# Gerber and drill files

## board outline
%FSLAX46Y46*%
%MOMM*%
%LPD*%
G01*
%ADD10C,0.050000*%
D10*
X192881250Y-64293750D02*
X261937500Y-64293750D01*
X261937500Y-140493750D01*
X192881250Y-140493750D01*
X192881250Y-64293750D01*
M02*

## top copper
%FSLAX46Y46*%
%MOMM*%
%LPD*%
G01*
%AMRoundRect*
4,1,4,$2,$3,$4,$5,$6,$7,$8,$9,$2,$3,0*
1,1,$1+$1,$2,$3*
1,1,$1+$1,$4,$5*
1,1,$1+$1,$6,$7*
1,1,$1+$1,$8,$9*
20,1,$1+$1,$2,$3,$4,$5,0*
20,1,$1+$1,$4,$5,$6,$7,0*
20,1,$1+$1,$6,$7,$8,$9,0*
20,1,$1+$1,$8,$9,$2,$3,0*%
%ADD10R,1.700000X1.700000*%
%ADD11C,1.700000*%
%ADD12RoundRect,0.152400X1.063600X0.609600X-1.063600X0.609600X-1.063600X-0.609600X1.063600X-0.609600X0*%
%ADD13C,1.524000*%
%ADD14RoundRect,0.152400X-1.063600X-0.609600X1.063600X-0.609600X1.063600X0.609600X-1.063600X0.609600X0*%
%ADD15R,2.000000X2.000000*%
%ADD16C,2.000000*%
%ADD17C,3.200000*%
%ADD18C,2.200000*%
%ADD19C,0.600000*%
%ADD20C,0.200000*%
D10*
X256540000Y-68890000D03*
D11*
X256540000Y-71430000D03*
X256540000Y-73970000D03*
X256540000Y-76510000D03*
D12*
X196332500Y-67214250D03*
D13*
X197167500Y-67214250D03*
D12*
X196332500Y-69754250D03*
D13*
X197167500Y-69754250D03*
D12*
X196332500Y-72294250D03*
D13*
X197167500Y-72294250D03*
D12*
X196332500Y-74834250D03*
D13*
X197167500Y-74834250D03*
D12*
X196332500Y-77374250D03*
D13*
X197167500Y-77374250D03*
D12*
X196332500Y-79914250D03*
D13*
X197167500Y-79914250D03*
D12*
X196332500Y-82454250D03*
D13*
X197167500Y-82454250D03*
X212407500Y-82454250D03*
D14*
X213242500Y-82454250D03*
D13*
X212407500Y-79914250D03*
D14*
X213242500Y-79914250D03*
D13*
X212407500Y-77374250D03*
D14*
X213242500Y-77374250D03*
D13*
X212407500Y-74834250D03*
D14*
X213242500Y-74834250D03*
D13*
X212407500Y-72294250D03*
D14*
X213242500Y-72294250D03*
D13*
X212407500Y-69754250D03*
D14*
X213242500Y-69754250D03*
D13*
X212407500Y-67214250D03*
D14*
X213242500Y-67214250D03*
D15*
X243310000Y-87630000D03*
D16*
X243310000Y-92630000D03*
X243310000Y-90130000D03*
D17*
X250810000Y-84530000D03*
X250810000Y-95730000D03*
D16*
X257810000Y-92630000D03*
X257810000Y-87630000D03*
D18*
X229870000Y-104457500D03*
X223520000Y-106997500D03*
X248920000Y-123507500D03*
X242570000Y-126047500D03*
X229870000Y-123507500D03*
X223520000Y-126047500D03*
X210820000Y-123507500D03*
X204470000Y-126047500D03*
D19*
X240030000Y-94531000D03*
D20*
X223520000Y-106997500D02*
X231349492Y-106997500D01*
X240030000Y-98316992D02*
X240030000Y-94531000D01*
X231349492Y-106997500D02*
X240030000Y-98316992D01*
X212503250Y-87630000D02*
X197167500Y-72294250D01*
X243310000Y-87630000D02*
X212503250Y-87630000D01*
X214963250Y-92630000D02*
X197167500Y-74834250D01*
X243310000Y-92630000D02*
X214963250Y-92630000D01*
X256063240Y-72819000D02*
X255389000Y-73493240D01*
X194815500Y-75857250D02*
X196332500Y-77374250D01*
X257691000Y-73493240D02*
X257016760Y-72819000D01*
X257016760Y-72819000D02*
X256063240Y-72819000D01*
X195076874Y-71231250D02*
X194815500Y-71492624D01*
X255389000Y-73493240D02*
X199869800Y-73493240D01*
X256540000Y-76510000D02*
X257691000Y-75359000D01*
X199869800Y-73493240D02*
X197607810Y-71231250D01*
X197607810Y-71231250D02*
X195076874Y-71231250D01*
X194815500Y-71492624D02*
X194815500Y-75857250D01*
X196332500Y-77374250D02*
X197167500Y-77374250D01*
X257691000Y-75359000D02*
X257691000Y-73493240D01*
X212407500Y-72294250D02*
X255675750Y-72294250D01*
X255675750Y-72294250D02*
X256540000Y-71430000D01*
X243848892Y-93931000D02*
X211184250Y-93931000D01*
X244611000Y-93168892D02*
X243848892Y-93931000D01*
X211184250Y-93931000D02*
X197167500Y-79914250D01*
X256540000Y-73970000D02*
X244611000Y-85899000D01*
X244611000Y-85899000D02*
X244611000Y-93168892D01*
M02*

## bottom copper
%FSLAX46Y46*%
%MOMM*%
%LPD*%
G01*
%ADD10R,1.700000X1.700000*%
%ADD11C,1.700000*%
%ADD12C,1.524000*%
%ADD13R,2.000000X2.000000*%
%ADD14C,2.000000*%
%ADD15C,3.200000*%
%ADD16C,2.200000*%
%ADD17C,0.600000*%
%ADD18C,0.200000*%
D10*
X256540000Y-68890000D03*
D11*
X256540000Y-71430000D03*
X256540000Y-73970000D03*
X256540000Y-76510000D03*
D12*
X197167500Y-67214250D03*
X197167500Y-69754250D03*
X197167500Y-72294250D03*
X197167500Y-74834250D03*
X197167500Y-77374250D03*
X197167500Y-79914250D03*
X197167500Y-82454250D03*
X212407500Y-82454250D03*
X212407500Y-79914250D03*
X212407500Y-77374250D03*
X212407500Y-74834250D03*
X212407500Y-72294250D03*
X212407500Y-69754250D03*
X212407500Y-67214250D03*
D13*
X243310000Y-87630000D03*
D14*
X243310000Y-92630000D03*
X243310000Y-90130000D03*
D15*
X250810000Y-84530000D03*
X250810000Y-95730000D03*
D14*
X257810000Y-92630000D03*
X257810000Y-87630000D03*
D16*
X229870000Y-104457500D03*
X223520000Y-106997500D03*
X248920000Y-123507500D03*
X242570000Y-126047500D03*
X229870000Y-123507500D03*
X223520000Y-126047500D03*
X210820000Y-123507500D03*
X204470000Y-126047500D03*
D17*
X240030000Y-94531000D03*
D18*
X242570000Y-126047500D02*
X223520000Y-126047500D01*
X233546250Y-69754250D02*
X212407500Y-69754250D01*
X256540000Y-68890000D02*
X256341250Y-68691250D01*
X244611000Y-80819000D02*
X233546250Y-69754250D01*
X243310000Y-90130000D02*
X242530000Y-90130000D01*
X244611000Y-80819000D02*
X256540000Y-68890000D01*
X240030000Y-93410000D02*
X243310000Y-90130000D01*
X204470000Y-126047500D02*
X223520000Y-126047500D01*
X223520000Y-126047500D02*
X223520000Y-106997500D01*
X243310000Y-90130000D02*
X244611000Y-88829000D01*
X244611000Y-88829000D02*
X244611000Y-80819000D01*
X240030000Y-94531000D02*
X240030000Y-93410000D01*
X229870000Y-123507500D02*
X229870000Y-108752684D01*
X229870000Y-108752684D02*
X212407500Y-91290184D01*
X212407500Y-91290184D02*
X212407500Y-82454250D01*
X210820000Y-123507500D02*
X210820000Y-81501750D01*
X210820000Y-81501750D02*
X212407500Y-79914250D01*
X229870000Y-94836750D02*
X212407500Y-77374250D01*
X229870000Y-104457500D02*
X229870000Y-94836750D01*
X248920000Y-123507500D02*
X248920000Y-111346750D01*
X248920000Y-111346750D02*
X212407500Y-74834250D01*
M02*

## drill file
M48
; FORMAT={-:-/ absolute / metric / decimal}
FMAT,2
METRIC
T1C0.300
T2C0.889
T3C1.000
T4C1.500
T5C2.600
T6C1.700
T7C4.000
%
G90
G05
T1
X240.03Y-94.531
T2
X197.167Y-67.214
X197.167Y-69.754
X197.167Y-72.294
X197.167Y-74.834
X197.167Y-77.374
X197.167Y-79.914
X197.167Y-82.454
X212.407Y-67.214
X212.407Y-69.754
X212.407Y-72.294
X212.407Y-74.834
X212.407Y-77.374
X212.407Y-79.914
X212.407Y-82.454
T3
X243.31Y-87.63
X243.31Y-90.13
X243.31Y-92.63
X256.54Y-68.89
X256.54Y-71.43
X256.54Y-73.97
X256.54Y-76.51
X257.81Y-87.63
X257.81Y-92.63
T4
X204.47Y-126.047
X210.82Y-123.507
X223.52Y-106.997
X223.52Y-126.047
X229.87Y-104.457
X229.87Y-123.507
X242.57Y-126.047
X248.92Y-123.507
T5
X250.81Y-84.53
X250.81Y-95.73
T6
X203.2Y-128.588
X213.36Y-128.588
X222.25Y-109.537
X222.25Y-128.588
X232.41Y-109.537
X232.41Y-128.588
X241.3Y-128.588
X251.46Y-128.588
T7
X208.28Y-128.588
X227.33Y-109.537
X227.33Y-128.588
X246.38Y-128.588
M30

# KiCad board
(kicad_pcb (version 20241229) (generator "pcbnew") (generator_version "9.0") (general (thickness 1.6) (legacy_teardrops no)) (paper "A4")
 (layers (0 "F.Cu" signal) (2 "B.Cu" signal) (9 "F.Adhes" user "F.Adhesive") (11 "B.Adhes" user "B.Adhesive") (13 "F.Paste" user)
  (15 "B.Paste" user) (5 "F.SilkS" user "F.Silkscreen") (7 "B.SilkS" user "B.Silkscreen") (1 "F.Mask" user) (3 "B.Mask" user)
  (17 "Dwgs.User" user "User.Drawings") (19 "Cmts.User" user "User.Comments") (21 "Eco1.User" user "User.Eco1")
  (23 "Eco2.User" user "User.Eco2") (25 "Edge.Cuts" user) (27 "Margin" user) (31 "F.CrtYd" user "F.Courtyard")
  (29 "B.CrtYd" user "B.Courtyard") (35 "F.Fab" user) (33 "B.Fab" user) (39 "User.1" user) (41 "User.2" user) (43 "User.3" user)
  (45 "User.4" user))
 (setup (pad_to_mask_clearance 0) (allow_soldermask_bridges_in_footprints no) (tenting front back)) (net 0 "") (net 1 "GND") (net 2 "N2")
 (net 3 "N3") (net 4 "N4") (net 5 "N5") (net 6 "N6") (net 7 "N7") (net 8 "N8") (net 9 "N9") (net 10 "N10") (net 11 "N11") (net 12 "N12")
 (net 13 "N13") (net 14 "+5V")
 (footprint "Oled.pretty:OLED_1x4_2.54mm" (layer "F.Cu") (at 256.54 68.89 -90)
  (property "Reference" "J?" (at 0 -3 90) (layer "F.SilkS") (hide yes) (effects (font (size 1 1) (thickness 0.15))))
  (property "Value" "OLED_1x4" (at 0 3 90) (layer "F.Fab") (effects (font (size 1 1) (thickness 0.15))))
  (pad "1" thru_hole rect (at 0 0 270) (size 1.7 1.7) (drill 1) (layers "*.Cu" "*.Mask") (remove_unused_layers no) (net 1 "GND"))
  (pad "2" thru_hole circle (at 2.54 0 270) (size 1.7 1.7) (drill 1) (layers "*.Cu" "*.Mask") (remove_unused_layers no) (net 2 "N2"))
  (pad "3" thru_hole circle (at 5.08 0 270) (size 1.7 1.7) (drill 1) (layers "*.Cu" "*.Mask") (remove_unused_layers no) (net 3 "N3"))
  (pad "4" thru_hole circle (at 7.62 0 270) (size 1.7 1.7) (drill 1) (layers "*.Cu" "*.Mask") (remove_unused_layers no) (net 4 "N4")))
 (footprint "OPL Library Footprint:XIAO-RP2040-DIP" (layer "F.Cu") (at 204.7875 74.83425)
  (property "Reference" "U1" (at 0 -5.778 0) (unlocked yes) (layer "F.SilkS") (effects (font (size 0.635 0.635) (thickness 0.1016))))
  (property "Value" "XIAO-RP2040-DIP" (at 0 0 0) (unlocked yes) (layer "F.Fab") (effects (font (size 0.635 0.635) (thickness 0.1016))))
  (pad "1" smd roundrect (at -8.455 -7.62 180) (size 2.432 1.524) (layers "F.Cu" "F.Mask") (roundrect_rratio 0.1) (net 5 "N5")
   (thermal_bridge_angle 45))
  (pad "1" thru_hole circle (at -7.62 -7.62 180) (size 1.524 1.524) (drill 0.889) (layers "*.Cu" "*.Mask") (remove_unused_layers no)
   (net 5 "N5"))
  (pad "2" smd roundrect (at -8.455 -5.08 180) (size 2.432 1.524) (layers "F.Cu" "F.Mask") (roundrect_rratio 0.1) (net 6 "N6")
   (thermal_bridge_angle 45))
  (pad "2" thru_hole circle (at -7.62 -5.08 180) (size 1.524 1.524) (drill 0.889) (layers "*.Cu" "*.Mask") (remove_unused_layers no)
   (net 6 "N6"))
  (pad "3" smd roundrect (at -8.455 -2.54 180) (size 2.432 1.524) (layers "F.Cu" "F.Mask") (roundrect_rratio 0.1) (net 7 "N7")
   (thermal_bridge_angle 45))
  (pad "3" thru_hole circle (at -7.62 -2.54 180) (size 1.524 1.524) (drill 0.889) (layers "*.Cu" "*.Mask") (remove_unused_layers no)
   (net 7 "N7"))
  (pad "4" smd roundrect (at -8.455 0 180) (size 2.432 1.524) (layers "F.Cu" "F.Mask") (roundrect_rratio 0.1) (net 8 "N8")
   (thermal_bridge_angle 45))
  (pad "4" thru_hole circle (at -7.62 0 180) (size 1.524 1.524) (drill 0.889) (layers "*.Cu" "*.Mask") (remove_unused_layers no)
   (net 8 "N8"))
  (pad "5" smd roundrect (at -8.455 2.54 180) (size 2.432 1.524) (layers "F.Cu" "F.Mask") (roundrect_rratio 0.1) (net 4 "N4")
   (thermal_bridge_angle 45))
  (pad "5" thru_hole circle (at -7.62 2.54 180) (size 1.524 1.524) (drill 0.889) (layers "*.Cu" "*.Mask") (remove_unused_layers no)
   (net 4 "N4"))
  (pad "6" smd roundrect (at -8.455 5.08 180) (size 2.432 1.524) (layers "F.Cu" "F.Mask") (roundrect_rratio 0.1) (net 3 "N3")
   (thermal_bridge_angle 45))
  (pad "6" thru_hole circle (at -7.62 5.08 180) (size 1.524 1.524) (drill 0.889) (layers "*.Cu" "*.Mask") (remove_unused_layers no)
   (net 3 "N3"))
  (pad "7" smd roundrect (at -8.455 7.62 180) (size 2.432 1.524) (layers "F.Cu" "F.Mask") (roundrect_rratio 0.1) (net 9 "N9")
   (thermal_bridge_angle 45))
  (pad "7" thru_hole circle (at -7.62 7.62 180) (size 1.524 1.524) (drill 0.889) (layers "*.Cu" "*.Mask") (remove_unused_layers no)
   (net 9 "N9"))
  (pad "8" thru_hole circle (at 7.62 7.62) (size 1.524 1.524) (drill 0.889) (layers "*.Cu" "*.Mask") (remove_unused_layers no)
   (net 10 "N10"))
  (pad "8" smd roundrect (at 8.455 7.62) (size 2.432 1.524) (layers "F.Cu" "F.Mask") (roundrect_rratio 0.1) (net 10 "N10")
   (thermal_bridge_angle 45))
  (pad "9" thru_hole circle (at 7.62 5.08) (size 1.524 1.524) (drill 0.889) (layers "*.Cu" "*.Mask") (remove_unused_layers no)
   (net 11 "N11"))
  (pad "9" smd roundrect (at 8.455 5.08) (size 2.432 1.524) (layers "F.Cu" "F.Mask") (roundrect_rratio 0.1) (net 11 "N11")
   (thermal_bridge_angle 45))
  (pad "10" thru_hole circle (at 7.62 2.54) (size 1.524 1.524) (drill 0.889) (layers "*.Cu" "*.Mask") (remove_unused_layers no)
   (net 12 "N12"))
  (pad "10" smd roundrect (at 8.455 2.54) (size 2.432 1.524) (layers "F.Cu" "F.Mask") (roundrect_rratio 0.1) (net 12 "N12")
   (thermal_bridge_angle 45))
  (pad "11" thru_hole circle (at 7.62 0) (size 1.524 1.524) (drill 0.889) (layers "*.Cu" "*.Mask") (remove_unused_layers no) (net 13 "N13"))
  (pad "11" smd roundrect (at 8.455 0) (size 2.432 1.524) (layers "F.Cu" "F.Mask") (roundrect_rratio 0.1) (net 13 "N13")
   (thermal_bridge_angle 45))
  (pad "12" thru_hole circle (at 7.62 -2.54) (size 1.524 1.524) (drill 0.889) (layers "*.Cu" "*.Mask") (remove_unused_layers no)
   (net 2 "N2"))
  (pad "12" smd roundrect (at 8.455 -2.54) (size 2.432 1.524) (layers "F.Cu" "F.Mask") (roundrect_rratio 0.1) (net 2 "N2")
   (thermal_bridge_angle 45))
  (pad "13" thru_hole circle (at 7.62 -5.08) (size 1.524 1.524) (drill 0.889) (layers "*.Cu" "*.Mask") (remove_unused_layers no)
   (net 1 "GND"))
  (pad "13" smd roundrect (at 8.455 -5.08) (size 2.432 1.524) (layers "F.Cu" "F.Mask") (roundrect_rratio 0.1) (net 1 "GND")
   (thermal_bridge_angle 45))
  (pad "14" thru_hole circle (at 7.62 -7.62) (size 1.524 1.524) (drill 0.889) (layers "*.Cu" "*.Mask") (remove_unused_layers no)
   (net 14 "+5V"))
  (pad "14" smd roundrect (at 8.455 -7.62) (size 2.432 1.524) (layers "F.Cu" "F.Mask") (roundrect_rratio 0.1) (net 14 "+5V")
   (thermal_bridge_angle 45)))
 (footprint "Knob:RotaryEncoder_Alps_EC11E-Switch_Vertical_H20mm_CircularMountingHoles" (layer "F.Cu") (at 243.31 87.63)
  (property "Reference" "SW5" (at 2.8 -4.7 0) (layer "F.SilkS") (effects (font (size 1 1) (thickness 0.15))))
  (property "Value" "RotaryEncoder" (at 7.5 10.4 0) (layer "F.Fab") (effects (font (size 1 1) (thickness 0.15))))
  (pad "A" thru_hole rect (at 0 0) (size 2 2) (drill 1) (layers "*.Cu" "*.Mask") (remove_unused_layers no) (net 7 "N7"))
  (pad "B" thru_hole circle (at 0 5) (size 2 2) (drill 1) (layers "*.Cu" "*.Mask") (remove_unused_layers no) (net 8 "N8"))
  (pad "C" thru_hole circle (at 0 2.5) (size 2 2) (drill 1) (layers "*.Cu" "*.Mask") (remove_unused_layers no) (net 1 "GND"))
  (pad "MP" thru_hole circle (at 7.5 -3.1) (size 3.2 3.2) (drill 2.6) (layers "*.Cu" "*.Mask") (remove_unused_layers no))
  (pad "MP" thru_hole circle (at 7.5 8.1) (size 3.2 3.2) (drill 2.6) (layers "*.Cu" "*.Mask") (remove_unused_layers no))
  (pad "S1" thru_hole circle (at 14.5 5) (size 2 2) (drill 1) (layers "*.Cu" "*.Mask") (remove_unused_layers no))
  (pad "S2" thru_hole circle (at 14.5 0) (size 2 2) (drill 1) (layers "*.Cu" "*.Mask") (remove_unused_layers no)))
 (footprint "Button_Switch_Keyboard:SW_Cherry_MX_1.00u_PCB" (layer "F.Cu") (at 229.87 104.4575)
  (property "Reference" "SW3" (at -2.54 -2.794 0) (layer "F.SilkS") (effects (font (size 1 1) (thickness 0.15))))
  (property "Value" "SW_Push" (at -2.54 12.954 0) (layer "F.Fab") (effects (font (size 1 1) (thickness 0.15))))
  (pad "" np_thru_hole circle (at -7.62 5.08) (size 1.7 1.7) (drill 1.7) (layers "*.Cu" "*.Mask"))
  (pad "" np_thru_hole circle (at -2.54 5.08) (size 4 4) (drill 4) (layers "*.Cu" "*.Mask"))
  (pad "" np_thru_hole circle (at 2.54 5.08) (size 1.7 1.7) (drill 1.7) (layers "*.Cu" "*.Mask"))
  (pad "1" thru_hole circle (at 0 0) (size 2.2 2.2) (drill 1.5) (layers "*.Cu" "*.Mask") (remove_unused_layers no) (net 12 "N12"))
  (pad "2" thru_hole circle (at -6.35 2.54) (size 2.2 2.2) (drill 1.5) (layers "*.Cu" "*.Mask") (remove_unused_layers no) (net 1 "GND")))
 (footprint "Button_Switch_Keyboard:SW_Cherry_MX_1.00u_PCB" (layer "F.Cu") (at 248.92 123.5075)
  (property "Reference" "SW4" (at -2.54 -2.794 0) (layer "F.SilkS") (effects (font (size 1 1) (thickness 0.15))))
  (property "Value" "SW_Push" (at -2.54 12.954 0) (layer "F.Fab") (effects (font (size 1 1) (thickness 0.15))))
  (pad "" np_thru_hole circle (at -7.62 5.08) (size 1.7 1.7) (drill 1.7) (layers "*.Cu" "*.Mask"))
  (pad "" np_thru_hole circle (at -2.54 5.08) (size 4 4) (drill 4) (layers "*.Cu" "*.Mask"))
  (pad "" np_thru_hole circle (at 2.54 5.08) (size 1.7 1.7) (drill 1.7) (layers "*.Cu" "*.Mask"))
  (pad "1" thru_hole circle (at 0 0) (size 2.2 2.2) (drill 1.5) (layers "*.Cu" "*.Mask") (remove_unused_layers no) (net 13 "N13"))
  (pad "2" thru_hole circle (at -6.35 2.54) (size 2.2 2.2) (drill 1.5) (layers "*.Cu" "*.Mask") (remove_unused_layers no) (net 1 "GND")))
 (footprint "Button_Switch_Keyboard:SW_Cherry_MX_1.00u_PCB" (layer "F.Cu") (at 229.87 123.5075)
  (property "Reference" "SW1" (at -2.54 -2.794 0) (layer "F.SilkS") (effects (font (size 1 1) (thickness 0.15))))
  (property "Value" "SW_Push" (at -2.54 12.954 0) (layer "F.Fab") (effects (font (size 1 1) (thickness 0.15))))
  (pad "" np_thru_hole circle (at -7.62 5.08) (size 1.7 1.7) (drill 1.7) (layers "*.Cu" "*.Mask"))
  (pad "" np_thru_hole circle (at -2.54 5.08) (size 4 4) (drill 4) (layers "*.Cu" "*.Mask"))
  (pad "" np_thru_hole circle (at 2.54 5.08) (size 1.7 1.7) (drill 1.7) (layers "*.Cu" "*.Mask"))
  (pad "1" thru_hole circle (at 0 0) (size 2.2 2.2) (drill 1.5) (layers "*.Cu" "*.Mask") (remove_unused_layers no) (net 10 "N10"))
  (pad "2" thru_hole circle (at -6.35 2.54) (size 2.2 2.2) (drill 1.5) (layers "*.Cu" "*.Mask") (remove_unused_layers no) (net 1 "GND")))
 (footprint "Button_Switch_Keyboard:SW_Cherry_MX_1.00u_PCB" (layer "F.Cu") (at 210.82 123.5075)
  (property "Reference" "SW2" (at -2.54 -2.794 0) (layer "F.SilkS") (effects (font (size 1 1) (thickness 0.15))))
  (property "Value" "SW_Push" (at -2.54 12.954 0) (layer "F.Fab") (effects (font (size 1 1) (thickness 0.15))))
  (pad "" np_thru_hole circle (at -7.62 5.08) (size 1.7 1.7) (drill 1.7) (layers "*.Cu" "*.Mask"))
  (pad "" np_thru_hole circle (at -2.54 5.08) (size 4 4) (drill 4) (layers "*.Cu" "*.Mask"))
  (pad "" np_thru_hole circle (at 2.54 5.08) (size 1.7 1.7) (drill 1.7) (layers "*.Cu" "*.Mask"))
  (pad "1" thru_hole circle (at 0 0) (size 2.2 2.2) (drill 1.5) (layers "*.Cu" "*.Mask") (remove_unused_layers no) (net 11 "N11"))
  (pad "2" thru_hole circle (at -6.35 2.54) (size 2.2 2.2) (drill 1.5) (layers "*.Cu" "*.Mask") (remove_unused_layers no) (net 1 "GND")))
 (gr_rect (start 192.88125 64.29375) (end 261.9375 140.49375) (stroke (width 0.05) (type default)) (fill no) (layer "Edge.Cuts"))
 (segment (start 223.52 106.9975) (end 231.349492 106.9975) (width 0.2) (layer "F.Cu") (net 1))
 (segment (start 240.03 98.316992) (end 240.03 94.531) (width 0.2) (layer "F.Cu") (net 1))
 (segment (start 231.349492 106.9975) (end 240.03 98.316992) (width 0.2) (layer "F.Cu") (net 1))
 (via (at 240.03 94.531) (size 0.6) (drill 0.3) (layers "F.Cu" "B.Cu") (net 1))
 (segment (start 242.57 126.0475) (end 223.52 126.0475) (width 0.2) (layer "B.Cu") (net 1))
 (segment (start 233.54625 69.75425) (end 212.4075 69.75425) (width 0.2) (layer "B.Cu") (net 1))
 (segment (start 256.54 68.89) (end 256.34125 68.69125) (width 0.2) (layer "B.Cu") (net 1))
 (segment (start 244.611 80.819) (end 233.54625 69.75425) (width 0.2) (layer "B.Cu") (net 1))
 (segment (start 243.31 90.13) (end 242.53 90.13) (width 0.2) (layer "B.Cu") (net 1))
 (segment (start 244.611 80.819) (end 256.54 68.89) (width 0.2) (layer "B.Cu") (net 1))
 (segment (start 240.03 93.41) (end 243.31 90.13) (width 0.2) (layer "B.Cu") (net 1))
 (segment (start 204.47 126.0475) (end 223.52 126.0475) (width 0.2) (layer "B.Cu") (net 1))
 (segment (start 223.52 126.0475) (end 223.52 106.9975) (width 0.2) (layer "B.Cu") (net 1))
 (segment (start 243.31 90.13) (end 244.611 88.829) (width 0.2) (layer "B.Cu") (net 1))
 (segment (start 244.611 88.829) (end 244.611 80.819) (width 0.2) (layer "B.Cu") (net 1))
 (segment (start 240.03 94.531) (end 240.03 93.41) (width 0.2) (layer "B.Cu") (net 1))
 (segment (start 229.87 123.5075) (end 229.87 108.752684) (width 0.2) (layer "B.Cu") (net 10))
 (segment (start 229.87 108.752684) (end 212.4075 91.290184) (width 0.2) (layer "B.Cu") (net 10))
 (segment (start 212.4075 91.290184) (end 212.4075 82.45425) (width 0.2) (layer "B.Cu") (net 10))
 (segment (start 210.82 123.5075) (end 210.82 81.50175) (width 0.2) (layer "B.Cu") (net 11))
 (segment (start 210.82 81.50175) (end 212.4075 79.91425) (width 0.2) (layer "B.Cu") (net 11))
 (segment (start 229.87 94.83675) (end 212.4075 77.37425) (width 0.2) (layer "B.Cu") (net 12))
 (segment (start 229.87 104.4575) (end 229.87 94.83675) (width 0.2) (layer "B.Cu") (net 12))
 (segment (start 248.92 123.5075) (end 248.92 111.34675) (width 0.2) (layer "B.Cu") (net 13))
 (segment (start 248.92 111.34675) (end 212.4075 74.83425) (width 0.2) (layer "B.Cu") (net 13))
 (segment (start 212.50325 87.63) (end 197.1675 72.29425) (width 0.2) (layer "F.Cu") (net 7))
 (segment (start 243.31 87.63) (end 212.50325 87.63) (width 0.2) (layer "F.Cu") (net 7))
 (segment (start 214.96325 92.63) (end 197.1675 74.83425) (width 0.2) (layer "F.Cu") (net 8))
 (segment (start 243.31 92.63) (end 214.96325 92.63) (width 0.2) (layer "F.Cu") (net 8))
 (segment (start 256.06324 72.819) (end 255.389 73.49324) (width 0.2) (layer "F.Cu") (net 4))
 (segment (start 194.8155 75.85725) (end 196.3325 77.37425) (width 0.2) (layer "F.Cu") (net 4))
 (segment (start 257.691 73.49324) (end 257.01676 72.819) (width 0.2) (layer "F.Cu") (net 4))
 (segment (start 257.01676 72.819) (end 256.06324 72.819) (width 0.2) (layer "F.Cu") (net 4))
 (segment (start 195.076874 71.23125) (end 194.8155 71.492624) (width 0.2) (layer "F.Cu") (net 4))
 (segment (start 255.389 73.49324) (end 199.8698 73.49324) (width 0.2) (layer "F.Cu") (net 4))
 (segment (start 256.54 76.51) (end 257.691 75.359) (width 0.2) (layer "F.Cu") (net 4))
 (segment (start 199.8698 73.49324) (end 197.60781 71.23125) (width 0.2) (layer "F.Cu") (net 4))
 (segment (start 197.60781 71.23125) (end 195.076874 71.23125) (width 0.2) (layer "F.Cu") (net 4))
 (segment (start 194.8155 71.492624) (end 194.8155 75.85725) (width 0.2) (layer "F.Cu") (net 4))
 (segment (start 196.3325 77.37425) (end 197.1675 77.37425) (width 0.2) (layer "F.Cu") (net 4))
 (segment (start 257.691 75.359) (end 257.691 73.49324) (width 0.2) (layer "F.Cu") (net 4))
 (segment (start 212.4075 72.29425) (end 255.67575 72.29425) (width 0.2) (layer "F.Cu") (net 2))
 (segment (start 255.67575 72.29425) (end 256.54 71.43) (width 0.2) (layer "F.Cu") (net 2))
 (segment (start 243.848892 93.931) (end 211.18425 93.931) (width 0.2) (layer "F.Cu") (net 3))
 (segment (start 244.611 93.168892) (end 243.848892 93.931) (width 0.2) (layer "F.Cu") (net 3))
 (segment (start 211.18425 93.931) (end 197.1675 79.91425) (width 0.2) (layer "F.Cu") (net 3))
 (segment (start 256.54 73.97) (end 244.611 85.899) (width 0.2) (layer "F.Cu") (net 3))
 (segment (start 244.611 85.899) (end 244.611 93.168892) (width 0.2) (layer "F.Cu") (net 3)))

